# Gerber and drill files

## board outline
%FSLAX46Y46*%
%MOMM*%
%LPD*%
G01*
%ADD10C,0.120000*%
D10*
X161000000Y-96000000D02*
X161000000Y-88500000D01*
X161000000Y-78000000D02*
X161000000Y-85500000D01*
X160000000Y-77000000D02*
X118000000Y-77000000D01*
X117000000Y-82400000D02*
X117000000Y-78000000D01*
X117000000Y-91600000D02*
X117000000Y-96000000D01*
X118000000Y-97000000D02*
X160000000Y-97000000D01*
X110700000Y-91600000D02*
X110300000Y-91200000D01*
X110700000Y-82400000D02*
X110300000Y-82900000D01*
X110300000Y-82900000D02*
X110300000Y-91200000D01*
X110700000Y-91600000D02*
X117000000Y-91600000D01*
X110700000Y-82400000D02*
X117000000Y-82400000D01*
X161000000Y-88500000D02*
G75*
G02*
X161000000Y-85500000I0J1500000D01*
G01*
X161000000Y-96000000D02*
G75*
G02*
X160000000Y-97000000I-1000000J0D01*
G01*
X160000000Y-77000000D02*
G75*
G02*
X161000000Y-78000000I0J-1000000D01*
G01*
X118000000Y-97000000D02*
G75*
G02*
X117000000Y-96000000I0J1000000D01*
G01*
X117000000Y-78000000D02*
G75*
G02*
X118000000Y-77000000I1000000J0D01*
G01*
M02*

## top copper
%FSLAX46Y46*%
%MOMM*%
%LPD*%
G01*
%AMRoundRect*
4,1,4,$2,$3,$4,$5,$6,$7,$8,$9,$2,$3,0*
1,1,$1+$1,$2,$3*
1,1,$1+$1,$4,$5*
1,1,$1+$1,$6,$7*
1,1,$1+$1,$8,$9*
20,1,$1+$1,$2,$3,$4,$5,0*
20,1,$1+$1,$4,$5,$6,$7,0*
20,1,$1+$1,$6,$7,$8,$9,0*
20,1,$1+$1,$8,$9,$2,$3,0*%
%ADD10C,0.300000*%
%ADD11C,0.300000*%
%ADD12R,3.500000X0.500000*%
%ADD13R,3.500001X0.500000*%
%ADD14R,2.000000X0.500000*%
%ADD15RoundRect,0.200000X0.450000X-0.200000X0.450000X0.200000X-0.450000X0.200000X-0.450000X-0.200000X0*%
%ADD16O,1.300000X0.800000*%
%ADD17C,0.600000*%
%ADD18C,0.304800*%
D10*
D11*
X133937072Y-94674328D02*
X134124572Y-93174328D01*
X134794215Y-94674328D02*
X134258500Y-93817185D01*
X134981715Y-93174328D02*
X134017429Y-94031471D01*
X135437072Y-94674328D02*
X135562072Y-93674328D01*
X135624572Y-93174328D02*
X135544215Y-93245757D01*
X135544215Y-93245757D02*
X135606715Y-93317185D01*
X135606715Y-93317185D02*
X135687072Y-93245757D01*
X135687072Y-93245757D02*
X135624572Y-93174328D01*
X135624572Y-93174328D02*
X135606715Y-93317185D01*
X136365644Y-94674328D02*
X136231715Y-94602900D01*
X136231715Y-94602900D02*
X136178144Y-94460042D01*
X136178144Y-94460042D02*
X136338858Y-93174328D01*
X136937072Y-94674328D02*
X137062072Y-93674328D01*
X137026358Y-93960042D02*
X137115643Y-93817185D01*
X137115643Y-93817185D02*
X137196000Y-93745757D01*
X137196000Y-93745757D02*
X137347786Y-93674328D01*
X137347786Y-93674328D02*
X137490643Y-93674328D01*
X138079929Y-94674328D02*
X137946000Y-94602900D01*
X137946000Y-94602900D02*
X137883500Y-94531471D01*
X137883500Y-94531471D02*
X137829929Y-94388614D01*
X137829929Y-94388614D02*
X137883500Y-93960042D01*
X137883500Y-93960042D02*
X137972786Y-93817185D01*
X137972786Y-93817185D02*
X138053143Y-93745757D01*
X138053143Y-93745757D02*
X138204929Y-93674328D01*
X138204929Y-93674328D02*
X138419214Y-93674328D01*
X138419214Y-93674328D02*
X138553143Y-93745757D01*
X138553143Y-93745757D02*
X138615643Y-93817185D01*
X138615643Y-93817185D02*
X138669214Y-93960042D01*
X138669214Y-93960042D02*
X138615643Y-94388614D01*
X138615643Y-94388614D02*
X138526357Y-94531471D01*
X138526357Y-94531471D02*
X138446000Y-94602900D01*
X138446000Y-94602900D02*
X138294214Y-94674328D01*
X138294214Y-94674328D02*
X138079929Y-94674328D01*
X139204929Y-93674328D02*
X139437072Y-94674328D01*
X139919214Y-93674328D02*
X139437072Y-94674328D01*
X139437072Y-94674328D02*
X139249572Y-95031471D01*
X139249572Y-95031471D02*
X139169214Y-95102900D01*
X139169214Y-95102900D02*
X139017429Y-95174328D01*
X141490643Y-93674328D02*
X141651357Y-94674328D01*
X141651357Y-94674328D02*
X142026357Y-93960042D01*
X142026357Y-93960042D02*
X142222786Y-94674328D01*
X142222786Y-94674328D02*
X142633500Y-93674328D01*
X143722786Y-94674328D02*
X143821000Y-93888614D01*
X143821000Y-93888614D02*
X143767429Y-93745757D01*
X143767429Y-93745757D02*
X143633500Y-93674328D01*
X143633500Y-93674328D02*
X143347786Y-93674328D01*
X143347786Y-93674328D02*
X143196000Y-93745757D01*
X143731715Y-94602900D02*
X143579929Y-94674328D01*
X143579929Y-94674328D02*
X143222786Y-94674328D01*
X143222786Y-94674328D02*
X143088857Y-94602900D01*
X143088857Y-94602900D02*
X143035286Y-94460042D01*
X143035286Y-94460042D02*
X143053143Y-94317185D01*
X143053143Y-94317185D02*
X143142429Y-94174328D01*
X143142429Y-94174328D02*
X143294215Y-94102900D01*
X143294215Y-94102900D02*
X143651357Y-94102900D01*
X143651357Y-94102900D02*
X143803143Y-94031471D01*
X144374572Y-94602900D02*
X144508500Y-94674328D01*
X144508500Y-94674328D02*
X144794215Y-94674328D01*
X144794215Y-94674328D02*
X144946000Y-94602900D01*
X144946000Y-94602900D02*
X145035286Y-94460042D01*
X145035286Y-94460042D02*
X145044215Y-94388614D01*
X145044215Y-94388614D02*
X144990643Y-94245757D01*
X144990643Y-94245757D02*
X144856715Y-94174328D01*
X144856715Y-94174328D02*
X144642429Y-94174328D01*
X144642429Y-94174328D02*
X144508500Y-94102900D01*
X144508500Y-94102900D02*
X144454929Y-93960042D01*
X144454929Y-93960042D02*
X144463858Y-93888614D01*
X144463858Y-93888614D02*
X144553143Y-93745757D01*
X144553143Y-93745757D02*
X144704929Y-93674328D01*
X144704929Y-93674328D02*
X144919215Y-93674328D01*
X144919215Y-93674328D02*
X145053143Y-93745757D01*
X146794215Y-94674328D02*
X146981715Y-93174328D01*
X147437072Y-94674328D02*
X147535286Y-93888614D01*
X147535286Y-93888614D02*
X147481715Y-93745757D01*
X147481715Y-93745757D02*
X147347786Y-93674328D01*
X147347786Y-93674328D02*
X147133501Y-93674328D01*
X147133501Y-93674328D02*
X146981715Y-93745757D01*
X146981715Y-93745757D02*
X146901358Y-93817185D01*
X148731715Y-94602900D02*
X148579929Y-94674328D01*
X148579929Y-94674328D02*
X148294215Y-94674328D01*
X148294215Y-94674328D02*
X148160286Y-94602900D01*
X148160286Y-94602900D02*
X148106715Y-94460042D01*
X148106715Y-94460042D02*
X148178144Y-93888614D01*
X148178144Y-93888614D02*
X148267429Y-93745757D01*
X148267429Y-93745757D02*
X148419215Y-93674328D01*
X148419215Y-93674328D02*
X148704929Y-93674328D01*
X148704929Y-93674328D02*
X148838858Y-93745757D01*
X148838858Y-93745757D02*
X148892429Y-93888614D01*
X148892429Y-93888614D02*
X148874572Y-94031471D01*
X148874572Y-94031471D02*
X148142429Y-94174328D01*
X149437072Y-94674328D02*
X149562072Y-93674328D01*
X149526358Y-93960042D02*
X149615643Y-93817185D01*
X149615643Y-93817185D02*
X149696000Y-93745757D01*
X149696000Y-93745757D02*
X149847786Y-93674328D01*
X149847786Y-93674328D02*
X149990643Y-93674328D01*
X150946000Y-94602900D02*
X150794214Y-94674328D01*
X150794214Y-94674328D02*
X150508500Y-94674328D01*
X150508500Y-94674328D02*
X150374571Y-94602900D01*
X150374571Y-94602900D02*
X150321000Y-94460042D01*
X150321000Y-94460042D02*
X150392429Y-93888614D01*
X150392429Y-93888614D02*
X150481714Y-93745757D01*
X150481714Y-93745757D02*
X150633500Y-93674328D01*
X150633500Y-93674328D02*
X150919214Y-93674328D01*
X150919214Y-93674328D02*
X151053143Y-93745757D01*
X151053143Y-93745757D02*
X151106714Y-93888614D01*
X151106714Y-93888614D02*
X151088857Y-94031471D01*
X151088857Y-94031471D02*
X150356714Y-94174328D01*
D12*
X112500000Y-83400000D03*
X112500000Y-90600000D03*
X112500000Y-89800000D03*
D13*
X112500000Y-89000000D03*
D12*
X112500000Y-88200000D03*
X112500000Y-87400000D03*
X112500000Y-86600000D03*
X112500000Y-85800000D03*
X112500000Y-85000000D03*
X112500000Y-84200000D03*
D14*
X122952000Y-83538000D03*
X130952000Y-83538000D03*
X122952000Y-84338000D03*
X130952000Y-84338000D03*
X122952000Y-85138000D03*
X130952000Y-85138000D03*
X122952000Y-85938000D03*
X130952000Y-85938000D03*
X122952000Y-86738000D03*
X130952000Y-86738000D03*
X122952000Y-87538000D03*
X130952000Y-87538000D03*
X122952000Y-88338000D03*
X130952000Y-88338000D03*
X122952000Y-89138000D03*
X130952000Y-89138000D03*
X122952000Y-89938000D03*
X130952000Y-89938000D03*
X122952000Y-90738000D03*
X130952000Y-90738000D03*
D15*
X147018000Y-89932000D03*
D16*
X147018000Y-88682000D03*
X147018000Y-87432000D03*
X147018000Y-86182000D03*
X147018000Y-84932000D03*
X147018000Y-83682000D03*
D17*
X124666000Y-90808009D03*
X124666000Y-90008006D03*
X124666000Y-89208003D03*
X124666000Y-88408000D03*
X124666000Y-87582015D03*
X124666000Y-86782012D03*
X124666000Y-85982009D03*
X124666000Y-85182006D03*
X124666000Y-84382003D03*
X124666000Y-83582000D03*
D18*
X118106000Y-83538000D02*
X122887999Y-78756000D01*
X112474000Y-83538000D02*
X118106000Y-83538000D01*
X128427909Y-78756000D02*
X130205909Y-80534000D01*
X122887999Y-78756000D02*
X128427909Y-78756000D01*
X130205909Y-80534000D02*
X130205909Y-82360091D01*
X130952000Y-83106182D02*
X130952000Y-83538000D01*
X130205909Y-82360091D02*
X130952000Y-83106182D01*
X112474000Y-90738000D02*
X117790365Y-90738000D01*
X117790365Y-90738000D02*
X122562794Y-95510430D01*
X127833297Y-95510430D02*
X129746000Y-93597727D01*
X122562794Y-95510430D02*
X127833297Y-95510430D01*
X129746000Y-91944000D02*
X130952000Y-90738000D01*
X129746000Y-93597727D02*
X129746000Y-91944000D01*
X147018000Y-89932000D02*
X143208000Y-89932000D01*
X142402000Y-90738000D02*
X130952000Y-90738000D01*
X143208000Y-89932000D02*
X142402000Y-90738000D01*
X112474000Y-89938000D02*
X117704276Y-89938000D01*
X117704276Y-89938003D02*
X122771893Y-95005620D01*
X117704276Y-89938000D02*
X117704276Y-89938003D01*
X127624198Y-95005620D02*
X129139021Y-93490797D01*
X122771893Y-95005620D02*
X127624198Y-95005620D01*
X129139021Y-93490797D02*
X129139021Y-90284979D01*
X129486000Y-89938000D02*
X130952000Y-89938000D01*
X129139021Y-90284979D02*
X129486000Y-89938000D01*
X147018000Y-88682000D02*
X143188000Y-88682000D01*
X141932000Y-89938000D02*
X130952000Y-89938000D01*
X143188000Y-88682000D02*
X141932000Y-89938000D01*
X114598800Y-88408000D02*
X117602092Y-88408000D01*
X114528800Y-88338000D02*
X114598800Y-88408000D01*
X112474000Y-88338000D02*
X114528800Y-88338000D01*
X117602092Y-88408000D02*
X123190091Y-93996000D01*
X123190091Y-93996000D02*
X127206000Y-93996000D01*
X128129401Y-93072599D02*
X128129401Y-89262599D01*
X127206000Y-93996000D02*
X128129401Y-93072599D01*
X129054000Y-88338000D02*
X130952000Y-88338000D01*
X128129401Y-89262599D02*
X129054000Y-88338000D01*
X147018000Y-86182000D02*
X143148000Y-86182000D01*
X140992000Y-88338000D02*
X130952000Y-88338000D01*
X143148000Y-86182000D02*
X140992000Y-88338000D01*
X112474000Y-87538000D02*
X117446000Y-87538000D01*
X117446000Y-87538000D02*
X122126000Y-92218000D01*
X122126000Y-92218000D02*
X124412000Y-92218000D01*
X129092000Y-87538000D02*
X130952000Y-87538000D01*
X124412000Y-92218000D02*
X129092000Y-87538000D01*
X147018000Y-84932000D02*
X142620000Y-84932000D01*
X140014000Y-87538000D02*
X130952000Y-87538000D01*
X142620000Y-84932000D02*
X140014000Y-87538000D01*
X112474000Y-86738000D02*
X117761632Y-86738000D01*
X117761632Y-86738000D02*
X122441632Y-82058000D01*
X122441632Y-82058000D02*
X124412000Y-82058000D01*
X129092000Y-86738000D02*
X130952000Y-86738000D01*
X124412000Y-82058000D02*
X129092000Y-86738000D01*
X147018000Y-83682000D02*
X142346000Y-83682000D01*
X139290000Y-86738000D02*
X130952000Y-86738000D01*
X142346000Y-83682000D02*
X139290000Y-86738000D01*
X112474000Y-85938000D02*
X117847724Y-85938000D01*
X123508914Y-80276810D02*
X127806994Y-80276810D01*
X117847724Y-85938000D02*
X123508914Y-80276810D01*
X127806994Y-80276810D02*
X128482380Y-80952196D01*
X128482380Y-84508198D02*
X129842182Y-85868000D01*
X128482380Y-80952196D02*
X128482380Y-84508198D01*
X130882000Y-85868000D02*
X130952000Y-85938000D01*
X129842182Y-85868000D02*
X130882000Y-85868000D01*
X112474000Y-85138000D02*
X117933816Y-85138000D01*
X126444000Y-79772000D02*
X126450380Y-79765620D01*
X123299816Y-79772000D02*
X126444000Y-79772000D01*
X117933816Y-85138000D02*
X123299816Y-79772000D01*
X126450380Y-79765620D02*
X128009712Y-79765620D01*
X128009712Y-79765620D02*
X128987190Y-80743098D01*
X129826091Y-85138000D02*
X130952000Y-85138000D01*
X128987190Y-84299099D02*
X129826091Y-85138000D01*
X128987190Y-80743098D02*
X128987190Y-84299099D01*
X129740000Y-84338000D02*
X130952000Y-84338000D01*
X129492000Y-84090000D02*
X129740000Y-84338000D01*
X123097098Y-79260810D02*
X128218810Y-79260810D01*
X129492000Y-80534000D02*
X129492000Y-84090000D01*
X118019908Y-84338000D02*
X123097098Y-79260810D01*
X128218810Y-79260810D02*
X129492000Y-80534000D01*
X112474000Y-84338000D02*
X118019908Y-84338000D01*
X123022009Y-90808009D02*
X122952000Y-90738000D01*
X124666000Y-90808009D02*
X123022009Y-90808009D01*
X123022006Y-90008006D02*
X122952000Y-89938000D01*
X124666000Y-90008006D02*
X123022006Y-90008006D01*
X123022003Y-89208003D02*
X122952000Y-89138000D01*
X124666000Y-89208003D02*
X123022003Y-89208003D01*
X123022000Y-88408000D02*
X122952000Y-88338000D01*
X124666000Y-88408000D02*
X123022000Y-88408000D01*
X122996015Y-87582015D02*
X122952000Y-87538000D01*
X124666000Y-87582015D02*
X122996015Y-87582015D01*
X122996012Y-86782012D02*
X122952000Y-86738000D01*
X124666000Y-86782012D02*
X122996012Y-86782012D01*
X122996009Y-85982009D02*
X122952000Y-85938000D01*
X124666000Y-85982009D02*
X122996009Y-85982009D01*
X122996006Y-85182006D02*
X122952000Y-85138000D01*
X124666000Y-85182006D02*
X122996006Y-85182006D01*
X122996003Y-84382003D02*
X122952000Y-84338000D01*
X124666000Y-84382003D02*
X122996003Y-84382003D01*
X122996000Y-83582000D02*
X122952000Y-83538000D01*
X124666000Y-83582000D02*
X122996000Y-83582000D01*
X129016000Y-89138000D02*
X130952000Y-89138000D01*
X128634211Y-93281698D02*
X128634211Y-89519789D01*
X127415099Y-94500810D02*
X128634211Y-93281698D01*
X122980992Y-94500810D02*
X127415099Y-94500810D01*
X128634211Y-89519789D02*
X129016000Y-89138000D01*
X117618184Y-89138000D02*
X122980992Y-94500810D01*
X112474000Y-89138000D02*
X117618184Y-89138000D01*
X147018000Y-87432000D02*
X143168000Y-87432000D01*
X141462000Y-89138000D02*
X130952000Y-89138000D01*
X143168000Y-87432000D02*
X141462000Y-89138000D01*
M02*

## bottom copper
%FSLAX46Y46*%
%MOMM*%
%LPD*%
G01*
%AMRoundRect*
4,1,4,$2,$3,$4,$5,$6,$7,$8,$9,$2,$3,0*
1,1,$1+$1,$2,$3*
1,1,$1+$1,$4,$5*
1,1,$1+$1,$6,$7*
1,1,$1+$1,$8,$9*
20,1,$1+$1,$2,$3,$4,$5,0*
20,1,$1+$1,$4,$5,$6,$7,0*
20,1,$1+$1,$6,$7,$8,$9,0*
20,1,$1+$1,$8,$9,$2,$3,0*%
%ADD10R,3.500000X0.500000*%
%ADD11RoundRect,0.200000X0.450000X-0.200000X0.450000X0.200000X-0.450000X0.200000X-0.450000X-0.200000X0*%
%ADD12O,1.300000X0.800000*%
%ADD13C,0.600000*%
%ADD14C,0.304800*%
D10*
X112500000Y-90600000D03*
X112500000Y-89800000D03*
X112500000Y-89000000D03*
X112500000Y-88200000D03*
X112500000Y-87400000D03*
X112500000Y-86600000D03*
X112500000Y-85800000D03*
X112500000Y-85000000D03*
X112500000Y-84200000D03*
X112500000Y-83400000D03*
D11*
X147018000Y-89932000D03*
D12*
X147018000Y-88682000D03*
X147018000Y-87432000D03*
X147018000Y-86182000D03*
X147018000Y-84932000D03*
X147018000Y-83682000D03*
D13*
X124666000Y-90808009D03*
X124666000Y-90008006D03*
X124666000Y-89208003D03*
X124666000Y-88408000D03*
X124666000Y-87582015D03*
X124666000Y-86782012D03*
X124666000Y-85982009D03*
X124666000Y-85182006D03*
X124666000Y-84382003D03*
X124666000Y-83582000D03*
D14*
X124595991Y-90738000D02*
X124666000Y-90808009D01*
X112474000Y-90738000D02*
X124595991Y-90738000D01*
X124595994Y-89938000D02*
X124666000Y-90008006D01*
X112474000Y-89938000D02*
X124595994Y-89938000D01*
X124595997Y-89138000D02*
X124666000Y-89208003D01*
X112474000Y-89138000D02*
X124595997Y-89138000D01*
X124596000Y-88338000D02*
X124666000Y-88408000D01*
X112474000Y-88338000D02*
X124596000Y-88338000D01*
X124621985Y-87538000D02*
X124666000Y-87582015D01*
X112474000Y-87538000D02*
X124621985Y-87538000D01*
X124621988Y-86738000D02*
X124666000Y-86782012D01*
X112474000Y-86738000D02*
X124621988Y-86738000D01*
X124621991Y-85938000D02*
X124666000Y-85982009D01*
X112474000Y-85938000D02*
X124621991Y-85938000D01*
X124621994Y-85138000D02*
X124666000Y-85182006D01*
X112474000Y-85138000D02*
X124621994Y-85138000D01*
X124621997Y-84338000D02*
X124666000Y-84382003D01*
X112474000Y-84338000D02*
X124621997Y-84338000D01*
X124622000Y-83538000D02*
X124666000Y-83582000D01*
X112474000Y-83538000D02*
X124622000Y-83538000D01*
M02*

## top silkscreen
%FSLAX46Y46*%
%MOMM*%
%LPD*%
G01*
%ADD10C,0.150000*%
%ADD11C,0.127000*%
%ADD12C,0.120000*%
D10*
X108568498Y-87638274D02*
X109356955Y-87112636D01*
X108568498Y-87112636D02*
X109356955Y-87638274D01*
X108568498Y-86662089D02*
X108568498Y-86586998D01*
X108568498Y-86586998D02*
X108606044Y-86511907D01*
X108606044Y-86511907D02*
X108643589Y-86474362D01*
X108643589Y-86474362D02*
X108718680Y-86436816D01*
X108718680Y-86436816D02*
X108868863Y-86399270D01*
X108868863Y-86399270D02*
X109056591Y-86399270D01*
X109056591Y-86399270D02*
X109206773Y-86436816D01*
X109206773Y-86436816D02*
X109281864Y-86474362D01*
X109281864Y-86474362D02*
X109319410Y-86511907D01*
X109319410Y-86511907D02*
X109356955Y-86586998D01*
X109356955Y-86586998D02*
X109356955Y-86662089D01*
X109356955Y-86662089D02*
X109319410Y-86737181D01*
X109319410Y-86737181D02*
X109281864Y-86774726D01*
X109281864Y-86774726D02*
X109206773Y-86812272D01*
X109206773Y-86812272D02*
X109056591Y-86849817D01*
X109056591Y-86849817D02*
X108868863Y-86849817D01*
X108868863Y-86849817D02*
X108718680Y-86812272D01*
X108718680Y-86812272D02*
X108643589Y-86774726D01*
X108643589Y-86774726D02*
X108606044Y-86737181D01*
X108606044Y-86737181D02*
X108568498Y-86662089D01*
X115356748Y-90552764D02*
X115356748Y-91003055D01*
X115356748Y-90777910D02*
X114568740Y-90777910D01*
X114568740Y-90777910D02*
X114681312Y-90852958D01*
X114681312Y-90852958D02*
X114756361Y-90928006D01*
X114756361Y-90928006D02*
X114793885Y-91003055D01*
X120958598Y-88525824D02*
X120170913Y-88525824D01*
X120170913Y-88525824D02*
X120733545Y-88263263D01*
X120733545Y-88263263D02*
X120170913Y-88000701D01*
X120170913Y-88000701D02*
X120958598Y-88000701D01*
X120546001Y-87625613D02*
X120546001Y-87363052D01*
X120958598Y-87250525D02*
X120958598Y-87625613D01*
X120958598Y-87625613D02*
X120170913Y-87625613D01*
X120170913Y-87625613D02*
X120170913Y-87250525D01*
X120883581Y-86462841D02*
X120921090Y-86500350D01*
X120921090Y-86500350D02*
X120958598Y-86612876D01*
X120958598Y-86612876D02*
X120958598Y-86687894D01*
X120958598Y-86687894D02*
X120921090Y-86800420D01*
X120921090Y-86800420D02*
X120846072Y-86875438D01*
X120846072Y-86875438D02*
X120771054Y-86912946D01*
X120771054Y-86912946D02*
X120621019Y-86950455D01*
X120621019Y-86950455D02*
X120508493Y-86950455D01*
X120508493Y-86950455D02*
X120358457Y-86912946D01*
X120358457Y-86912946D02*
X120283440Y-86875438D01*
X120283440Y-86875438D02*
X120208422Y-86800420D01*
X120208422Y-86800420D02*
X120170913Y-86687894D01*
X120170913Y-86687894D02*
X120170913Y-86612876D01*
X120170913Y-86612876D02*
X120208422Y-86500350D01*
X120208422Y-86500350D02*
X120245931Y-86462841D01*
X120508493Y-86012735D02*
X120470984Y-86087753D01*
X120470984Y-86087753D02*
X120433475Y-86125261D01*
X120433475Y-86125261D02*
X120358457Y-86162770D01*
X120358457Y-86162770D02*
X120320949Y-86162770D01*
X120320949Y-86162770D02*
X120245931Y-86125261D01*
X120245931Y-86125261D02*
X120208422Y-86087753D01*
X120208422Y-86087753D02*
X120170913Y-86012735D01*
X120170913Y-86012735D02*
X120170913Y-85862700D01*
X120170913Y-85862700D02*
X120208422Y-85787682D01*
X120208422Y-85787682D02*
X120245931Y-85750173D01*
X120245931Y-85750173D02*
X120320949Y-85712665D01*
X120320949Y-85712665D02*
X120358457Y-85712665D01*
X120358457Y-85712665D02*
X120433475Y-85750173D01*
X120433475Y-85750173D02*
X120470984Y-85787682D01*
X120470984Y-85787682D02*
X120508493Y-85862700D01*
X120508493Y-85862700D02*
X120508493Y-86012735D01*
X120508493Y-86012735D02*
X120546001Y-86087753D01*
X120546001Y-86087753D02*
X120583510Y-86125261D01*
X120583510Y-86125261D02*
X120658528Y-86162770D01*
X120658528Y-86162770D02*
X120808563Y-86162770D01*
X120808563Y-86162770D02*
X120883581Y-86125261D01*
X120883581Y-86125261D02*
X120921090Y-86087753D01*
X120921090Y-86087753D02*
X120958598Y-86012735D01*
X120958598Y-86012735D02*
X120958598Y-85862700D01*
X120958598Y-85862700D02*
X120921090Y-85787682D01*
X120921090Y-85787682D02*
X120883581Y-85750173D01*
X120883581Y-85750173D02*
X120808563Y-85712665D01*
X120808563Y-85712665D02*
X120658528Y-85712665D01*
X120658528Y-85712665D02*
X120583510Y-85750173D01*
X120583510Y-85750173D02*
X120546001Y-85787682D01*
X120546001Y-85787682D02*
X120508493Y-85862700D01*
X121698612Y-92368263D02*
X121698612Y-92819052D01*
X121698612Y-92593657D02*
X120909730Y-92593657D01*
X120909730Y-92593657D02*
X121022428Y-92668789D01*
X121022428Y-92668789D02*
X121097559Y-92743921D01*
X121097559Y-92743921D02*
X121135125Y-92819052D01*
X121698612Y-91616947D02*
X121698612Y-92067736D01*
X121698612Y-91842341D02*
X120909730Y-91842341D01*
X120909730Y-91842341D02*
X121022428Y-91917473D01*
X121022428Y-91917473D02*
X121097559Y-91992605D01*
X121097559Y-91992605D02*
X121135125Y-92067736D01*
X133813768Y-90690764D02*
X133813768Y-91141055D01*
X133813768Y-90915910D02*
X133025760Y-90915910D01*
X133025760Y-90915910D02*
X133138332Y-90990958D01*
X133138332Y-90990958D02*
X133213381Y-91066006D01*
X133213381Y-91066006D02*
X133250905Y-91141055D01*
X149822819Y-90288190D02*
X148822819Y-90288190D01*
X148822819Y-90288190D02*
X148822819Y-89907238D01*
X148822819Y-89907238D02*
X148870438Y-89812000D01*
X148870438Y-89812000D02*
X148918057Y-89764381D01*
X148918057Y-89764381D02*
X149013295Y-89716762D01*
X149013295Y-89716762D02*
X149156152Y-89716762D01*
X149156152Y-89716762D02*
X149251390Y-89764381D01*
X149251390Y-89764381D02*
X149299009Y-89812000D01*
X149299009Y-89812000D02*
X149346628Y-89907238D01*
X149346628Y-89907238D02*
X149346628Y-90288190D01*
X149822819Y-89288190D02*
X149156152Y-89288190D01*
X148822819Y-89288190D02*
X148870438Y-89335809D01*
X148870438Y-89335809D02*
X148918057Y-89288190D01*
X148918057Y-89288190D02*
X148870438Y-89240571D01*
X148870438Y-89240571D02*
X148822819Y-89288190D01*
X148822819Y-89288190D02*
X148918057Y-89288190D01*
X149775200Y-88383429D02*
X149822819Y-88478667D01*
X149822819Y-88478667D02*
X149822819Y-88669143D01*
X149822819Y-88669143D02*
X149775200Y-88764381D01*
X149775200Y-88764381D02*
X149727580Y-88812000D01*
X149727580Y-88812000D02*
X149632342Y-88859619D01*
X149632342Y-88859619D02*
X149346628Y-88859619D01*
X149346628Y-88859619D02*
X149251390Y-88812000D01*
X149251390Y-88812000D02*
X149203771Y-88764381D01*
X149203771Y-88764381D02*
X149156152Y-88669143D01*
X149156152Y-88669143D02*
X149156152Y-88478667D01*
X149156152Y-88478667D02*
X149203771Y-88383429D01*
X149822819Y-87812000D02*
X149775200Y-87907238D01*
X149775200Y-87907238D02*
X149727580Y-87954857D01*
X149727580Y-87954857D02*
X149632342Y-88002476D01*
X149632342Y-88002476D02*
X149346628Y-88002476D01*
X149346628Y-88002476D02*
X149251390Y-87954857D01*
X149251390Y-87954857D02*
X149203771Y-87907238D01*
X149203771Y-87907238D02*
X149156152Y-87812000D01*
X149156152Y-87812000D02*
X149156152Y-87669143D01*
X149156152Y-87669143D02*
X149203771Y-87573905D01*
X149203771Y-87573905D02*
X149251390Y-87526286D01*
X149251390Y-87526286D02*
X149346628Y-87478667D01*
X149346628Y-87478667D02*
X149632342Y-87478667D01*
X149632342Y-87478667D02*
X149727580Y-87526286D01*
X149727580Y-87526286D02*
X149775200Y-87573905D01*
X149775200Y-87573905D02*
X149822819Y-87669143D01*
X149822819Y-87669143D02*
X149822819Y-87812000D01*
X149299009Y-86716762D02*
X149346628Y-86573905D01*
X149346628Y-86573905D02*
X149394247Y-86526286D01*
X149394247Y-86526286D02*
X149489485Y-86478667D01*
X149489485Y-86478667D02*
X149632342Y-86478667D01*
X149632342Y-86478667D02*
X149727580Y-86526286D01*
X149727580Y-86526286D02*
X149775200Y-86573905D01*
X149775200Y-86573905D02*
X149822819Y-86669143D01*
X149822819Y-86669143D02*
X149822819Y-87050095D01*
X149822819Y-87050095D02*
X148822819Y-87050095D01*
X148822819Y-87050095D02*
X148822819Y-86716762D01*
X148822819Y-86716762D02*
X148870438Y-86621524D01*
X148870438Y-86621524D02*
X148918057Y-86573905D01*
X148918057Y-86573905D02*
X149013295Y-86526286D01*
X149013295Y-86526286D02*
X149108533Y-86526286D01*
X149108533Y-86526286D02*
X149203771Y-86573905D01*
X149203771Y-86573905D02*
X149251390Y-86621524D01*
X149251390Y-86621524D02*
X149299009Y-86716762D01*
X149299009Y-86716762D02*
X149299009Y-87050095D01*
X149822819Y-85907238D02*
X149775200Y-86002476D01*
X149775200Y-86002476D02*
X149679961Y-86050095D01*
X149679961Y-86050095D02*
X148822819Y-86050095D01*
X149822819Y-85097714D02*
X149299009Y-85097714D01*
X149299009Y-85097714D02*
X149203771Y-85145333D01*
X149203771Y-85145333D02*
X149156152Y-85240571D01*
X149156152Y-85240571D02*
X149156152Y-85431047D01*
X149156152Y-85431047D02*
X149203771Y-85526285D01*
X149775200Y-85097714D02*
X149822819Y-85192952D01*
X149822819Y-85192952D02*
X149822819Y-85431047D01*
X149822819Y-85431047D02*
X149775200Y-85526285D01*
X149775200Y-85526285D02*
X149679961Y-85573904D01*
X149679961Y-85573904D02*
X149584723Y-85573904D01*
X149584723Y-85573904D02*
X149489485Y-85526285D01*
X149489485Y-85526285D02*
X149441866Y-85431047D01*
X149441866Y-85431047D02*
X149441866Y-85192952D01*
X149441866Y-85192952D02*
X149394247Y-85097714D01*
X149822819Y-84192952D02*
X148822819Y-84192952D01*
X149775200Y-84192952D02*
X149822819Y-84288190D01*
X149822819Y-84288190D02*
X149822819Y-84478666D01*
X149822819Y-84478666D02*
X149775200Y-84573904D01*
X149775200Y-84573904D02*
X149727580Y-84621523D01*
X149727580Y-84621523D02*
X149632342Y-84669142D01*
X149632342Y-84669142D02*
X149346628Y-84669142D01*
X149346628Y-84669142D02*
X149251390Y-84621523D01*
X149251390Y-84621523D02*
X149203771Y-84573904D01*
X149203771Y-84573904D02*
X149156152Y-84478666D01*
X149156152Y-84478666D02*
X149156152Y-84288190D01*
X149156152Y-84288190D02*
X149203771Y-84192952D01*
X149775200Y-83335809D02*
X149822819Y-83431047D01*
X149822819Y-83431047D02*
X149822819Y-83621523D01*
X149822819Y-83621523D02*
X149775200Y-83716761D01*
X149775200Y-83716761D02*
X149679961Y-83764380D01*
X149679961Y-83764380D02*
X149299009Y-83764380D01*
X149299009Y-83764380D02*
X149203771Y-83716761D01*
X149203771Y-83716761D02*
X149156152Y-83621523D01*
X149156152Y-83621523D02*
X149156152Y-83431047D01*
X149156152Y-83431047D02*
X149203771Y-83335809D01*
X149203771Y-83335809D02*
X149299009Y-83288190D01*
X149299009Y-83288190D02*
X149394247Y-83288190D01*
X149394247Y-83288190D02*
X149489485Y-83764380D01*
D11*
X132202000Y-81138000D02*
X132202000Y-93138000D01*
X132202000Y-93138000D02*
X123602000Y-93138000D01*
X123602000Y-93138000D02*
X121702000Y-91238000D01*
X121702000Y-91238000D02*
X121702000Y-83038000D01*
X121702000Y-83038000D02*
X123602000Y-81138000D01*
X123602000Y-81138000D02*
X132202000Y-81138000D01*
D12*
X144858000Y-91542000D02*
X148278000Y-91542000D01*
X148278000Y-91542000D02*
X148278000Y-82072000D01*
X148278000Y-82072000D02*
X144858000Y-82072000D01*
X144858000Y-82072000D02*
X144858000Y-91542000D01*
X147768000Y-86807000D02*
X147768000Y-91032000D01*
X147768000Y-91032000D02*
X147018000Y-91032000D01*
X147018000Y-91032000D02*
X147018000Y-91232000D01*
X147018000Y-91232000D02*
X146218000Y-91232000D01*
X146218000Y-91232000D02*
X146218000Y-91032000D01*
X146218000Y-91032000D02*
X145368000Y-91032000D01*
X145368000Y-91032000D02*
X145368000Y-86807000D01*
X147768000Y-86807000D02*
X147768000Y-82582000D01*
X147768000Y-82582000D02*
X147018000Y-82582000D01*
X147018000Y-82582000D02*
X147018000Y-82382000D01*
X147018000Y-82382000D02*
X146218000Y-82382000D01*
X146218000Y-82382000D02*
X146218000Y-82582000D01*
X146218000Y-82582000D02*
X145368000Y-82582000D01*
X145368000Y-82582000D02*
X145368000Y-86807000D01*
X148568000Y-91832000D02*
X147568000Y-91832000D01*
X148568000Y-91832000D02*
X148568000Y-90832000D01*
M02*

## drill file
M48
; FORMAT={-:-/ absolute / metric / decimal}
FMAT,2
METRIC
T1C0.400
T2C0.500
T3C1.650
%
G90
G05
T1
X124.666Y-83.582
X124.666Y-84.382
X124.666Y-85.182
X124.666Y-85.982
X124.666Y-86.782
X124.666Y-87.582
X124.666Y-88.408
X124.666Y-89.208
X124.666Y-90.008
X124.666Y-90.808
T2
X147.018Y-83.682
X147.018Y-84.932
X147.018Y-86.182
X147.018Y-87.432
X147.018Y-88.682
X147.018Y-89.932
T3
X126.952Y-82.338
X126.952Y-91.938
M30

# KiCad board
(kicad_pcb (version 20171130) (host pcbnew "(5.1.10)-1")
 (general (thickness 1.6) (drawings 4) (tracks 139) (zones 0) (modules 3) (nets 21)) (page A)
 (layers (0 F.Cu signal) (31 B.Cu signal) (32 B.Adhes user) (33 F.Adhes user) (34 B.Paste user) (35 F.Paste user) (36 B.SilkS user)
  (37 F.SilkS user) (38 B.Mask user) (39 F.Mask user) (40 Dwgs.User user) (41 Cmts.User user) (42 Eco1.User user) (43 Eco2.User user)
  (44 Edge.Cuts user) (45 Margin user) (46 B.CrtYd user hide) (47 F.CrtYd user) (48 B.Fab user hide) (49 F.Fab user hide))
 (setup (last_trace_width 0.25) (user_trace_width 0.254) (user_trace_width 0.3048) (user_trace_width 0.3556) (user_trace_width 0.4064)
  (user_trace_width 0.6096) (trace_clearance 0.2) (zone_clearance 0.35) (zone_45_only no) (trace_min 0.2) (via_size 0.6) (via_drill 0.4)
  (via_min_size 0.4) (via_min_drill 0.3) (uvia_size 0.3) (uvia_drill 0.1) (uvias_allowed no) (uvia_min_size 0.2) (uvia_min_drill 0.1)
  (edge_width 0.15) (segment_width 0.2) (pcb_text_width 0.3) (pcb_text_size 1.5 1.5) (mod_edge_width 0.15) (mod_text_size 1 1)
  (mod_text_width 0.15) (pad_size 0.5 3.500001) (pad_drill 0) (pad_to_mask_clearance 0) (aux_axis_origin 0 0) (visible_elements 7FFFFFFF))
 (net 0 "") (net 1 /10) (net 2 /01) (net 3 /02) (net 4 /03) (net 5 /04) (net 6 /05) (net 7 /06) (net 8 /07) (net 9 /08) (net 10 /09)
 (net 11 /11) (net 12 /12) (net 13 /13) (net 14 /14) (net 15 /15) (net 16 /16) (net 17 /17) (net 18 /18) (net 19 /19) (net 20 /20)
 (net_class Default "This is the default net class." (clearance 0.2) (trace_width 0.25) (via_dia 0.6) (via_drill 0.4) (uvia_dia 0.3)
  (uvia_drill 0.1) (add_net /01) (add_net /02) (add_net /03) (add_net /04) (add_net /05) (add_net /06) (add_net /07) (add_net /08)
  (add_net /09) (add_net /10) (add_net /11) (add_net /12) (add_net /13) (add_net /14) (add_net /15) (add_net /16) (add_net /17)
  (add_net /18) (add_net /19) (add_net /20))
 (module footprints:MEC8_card (layer F.Cu) (at 112.5 87 90)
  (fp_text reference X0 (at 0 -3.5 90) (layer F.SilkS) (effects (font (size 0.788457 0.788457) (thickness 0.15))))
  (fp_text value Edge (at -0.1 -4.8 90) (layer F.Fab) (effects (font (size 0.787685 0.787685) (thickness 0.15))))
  (fp_line (start -9 48.5) (end -1.5 48.5) (layer Edge.Cuts) (width 0.12))
  (fp_line (start 9 48.5) (end 1.5 48.5) (layer Edge.Cuts) (width 0.12))
  (fp_line (start 10 47.5) (end 10 5.5) (layer Edge.Cuts) (width 0.12))
  (fp_line (start 4.6 4.5) (end 9 4.5) (layer Edge.Cuts) (width 0.12))
  (fp_line (start -4.6 4.5) (end -9 4.5) (layer Edge.Cuts) (width 0.12))
  (fp_line (start -10 5.5) (end -10 47.5) (layer Edge.Cuts) (width 0.12))
  (fp_line (start -4.6 -1.8) (end -4.2 -2.2) (layer Edge.Cuts) (width 0.12))
  (fp_line (start 4.6 -1.8) (end 4.1 -2.2) (layer Edge.Cuts) (width 0.12))
  (fp_line (start 4.1 -2.2) (end -4.2 -2.2) (layer Edge.Cuts) (width 0.12))
  (fp_line (start -4.6 -1.8) (end -4.6 4.5) (layer Edge.Cuts) (width 0.12))
  (fp_line (start 4.6 -1.8) (end 4.6 4.5) (layer Edge.Cuts) (width 0.12))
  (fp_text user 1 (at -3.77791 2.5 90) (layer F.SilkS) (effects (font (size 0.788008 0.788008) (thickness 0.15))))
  (fp_arc (start 0 48.5) (end 1.5 48.5) (angle -180) (layer Edge.Cuts) (width 0.12))
  (fp_arc (start -9 47.5) (end -10 47.5) (angle -90) (layer Edge.Cuts) (width 0.12))
  (fp_arc (start 9 47.5) (end 9 48.5) (angle -90) (layer Edge.Cuts) (width 0.12))
  (fp_arc (start -9 5.5) (end -9 4.5) (angle -90) (layer Edge.Cuts) (width 0.12))
  (fp_arc (start 9 5.5) (end 10 5.5) (angle -90) (layer Edge.Cuts) (width 0.12))
  (pad 10 smd rect (at 3.6 0 90) (size 0.5 3.5) (layers F.Cu F.Paste F.Mask) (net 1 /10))
  (pad 1 smd rect (at -3.6 0 90) (size 0.5 3.5) (layers F.Cu F.Paste F.Mask) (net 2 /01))
  (pad 2 smd rect (at -2.8 0 90) (size 0.5 3.5) (layers F.Cu F.Paste F.Mask) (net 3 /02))
  (pad 3 smd rect (at -2 0 90) (size 0.5 3.500001) (layers F.Cu F.Paste F.Mask) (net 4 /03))
  (pad 4 smd rect (at -1.2 0 90) (size 0.5 3.5) (layers F.Cu F.Paste F.Mask) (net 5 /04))
  (pad 5 smd rect (at -0.4 0 90) (size 0.5 3.5) (layers F.Cu F.Paste F.Mask) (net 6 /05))
  (pad 6 smd rect (at 0.4 0 90) (size 0.5 3.5) (layers F.Cu F.Paste F.Mask) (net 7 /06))
  (pad 7 smd rect (at 1.2 0 90) (size 0.5 3.5) (layers F.Cu F.Paste F.Mask) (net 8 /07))
  (pad 8 smd rect (at 2 0 90) (size 0.5 3.5) (layers F.Cu F.Paste F.Mask) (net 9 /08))
  (pad 9 smd rect (at 2.8 0 90) (size 0.5 3.5) (layers F.Cu F.Paste F.Mask) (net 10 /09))
  (pad 11 smd rect (at -3.6 0 90) (size 0.5 3.5) (layers B.Cu B.Paste B.Mask) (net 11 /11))
  (pad 12 smd rect (at -2.8 0 90) (size 0.5 3.5) (layers B.Cu B.Paste B.Mask) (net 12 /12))
  (pad 13 smd rect (at -2 0 90) (size 0.5 3.5) (layers B.Cu B.Paste B.Mask) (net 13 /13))
  (pad 14 smd rect (at -1.2 0 90) (size 0.5 3.5) (layers B.Cu B.Paste B.Mask) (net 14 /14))
  (pad 15 smd rect (at -0.4 0 90) (size 0.5 3.5) (layers B.Cu B.Paste B.Mask) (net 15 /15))
  (pad 16 smd rect (at 0.4 0 90) (size 0.5 3.5) (layers B.Cu B.Paste B.Mask) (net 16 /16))
  (pad 17 smd rect (at 1.2 0 90) (size 0.5 3.5) (layers B.Cu B.Paste B.Mask) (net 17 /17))
  (pad 18 smd rect (at 2 0 90) (size 0.5 3.5) (layers B.Cu B.Paste B.Mask) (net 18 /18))
  (pad 19 smd rect (at 2.8 0 90) (size 0.5 3.5) (layers B.Cu B.Paste B.Mask) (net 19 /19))
  (pad 20 smd rect (at 3.6 0 90) (size 0.5 3.5) (layers B.Cu B.Paste B.Mask) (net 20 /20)))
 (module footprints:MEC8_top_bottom (layer F.Cu) (at 126.952 87.138 90)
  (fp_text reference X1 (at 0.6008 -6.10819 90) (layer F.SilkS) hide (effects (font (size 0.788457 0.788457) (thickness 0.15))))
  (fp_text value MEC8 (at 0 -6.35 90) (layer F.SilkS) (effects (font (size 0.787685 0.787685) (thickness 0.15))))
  (fp_line (start 6 5.25) (end -6 5.25) (layer F.SilkS) (width 0.127))
  (fp_line (start -6 5.25) (end -6 -3.35) (layer F.SilkS) (width 0.127))
  (fp_line (start -6 -3.35) (end -4.1 -5.25) (layer F.SilkS) (width 0.127))
  (fp_line (start -4.1 -5.25) (end 4.1 -5.25) (layer F.SilkS) (width 0.127))
  (fp_line (start 4.1 -5.25) (end 6 -3.35) (layer F.SilkS) (width 0.127))
  (fp_line (start 6 -3.35) (end 6 5.25) (layer F.SilkS) (width 0.127))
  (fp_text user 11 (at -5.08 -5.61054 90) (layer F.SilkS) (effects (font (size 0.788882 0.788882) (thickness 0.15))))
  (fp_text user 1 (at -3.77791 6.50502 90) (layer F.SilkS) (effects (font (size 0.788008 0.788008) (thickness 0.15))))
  (pad None np_thru_hole circle (at 4.8 0 90) (size 1.65 1.65) (drill 1.65) (layers *.Cu *.Mask))
  (pad None np_thru_hole circle (at -4.8 0 90) (size 1.65 1.65) (drill 1.65) (layers *.Cu *.Mask))
  (pad 20 smd rect (at 3.6 -4 90) (size 0.5 2) (layers F.Cu F.Paste F.Mask) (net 20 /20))
  (pad 10 smd rect (at 3.6 4 90) (size 0.5 2) (layers F.Cu F.Paste F.Mask) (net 1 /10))
  (pad 19 smd rect (at 2.8 -4 90) (size 0.5 2) (layers F.Cu F.Paste F.Mask) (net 19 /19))
  (pad 9 smd rect (at 2.8 4 90) (size 0.5 2) (layers F.Cu F.Paste F.Mask) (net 10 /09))
  (pad 18 smd rect (at 2 -4 90) (size 0.5 2) (layers F.Cu F.Paste F.Mask) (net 18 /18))
  (pad 8 smd rect (at 2 4 90) (size 0.5 2) (layers F.Cu F.Paste F.Mask) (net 9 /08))
  (pad 17 smd rect (at 1.2 -4 90) (size 0.5 2) (layers F.Cu F.Paste F.Mask) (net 17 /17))
  (pad 7 smd rect (at 1.2 4 90) (size 0.5 2) (layers F.Cu F.Paste F.Mask) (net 8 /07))
  (pad 16 smd rect (at 0.4 -4 90) (size 0.5 2) (layers F.Cu F.Paste F.Mask) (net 16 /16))
  (pad 6 smd rect (at 0.4 4 90) (size 0.5 2) (layers F.Cu F.Paste F.Mask) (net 7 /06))
  (pad 15 smd rect (at -0.4 -4 90) (size 0.5 2) (layers F.Cu F.Paste F.Mask) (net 15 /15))
  (pad 5 smd rect (at -0.4 4 90) (size 0.5 2) (layers F.Cu F.Paste F.Mask) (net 6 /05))
  (pad 14 smd rect (at -1.2 -4 90) (size 0.5 2) (layers F.Cu F.Paste F.Mask) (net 14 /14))
  (pad 4 smd rect (at -1.2 4 90) (size 0.5 2) (layers F.Cu F.Paste F.Mask) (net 5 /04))
  (pad 13 smd rect (at -2 -4 90) (size 0.5 2) (layers F.Cu F.Paste F.Mask) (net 13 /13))
  (pad 3 smd rect (at -2 4 90) (size 0.5 2) (layers F.Cu F.Paste F.Mask) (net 4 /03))
  (pad 12 smd rect (at -2.8 -4 90) (size 0.5 2) (layers F.Cu F.Paste F.Mask) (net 12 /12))
  (pad 2 smd rect (at -2.8 4 90) (size 0.5 2) (layers F.Cu F.Paste F.Mask) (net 3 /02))
  (pad 11 smd rect (at -3.6 -4 90) (size 0.5 2) (layers F.Cu F.Paste F.Mask) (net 11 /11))
  (pad 1 smd rect (at -3.6 4 90) (size 0.5 2) (layers F.Cu F.Paste F.Mask) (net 2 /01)))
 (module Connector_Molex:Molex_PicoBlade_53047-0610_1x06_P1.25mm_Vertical (layer F.Cu) (at 147.018 89.932 90)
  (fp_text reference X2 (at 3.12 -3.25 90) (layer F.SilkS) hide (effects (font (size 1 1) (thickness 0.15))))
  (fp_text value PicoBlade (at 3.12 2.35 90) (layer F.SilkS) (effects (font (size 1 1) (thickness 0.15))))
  (fp_line (start -1.61 -2.16) (end -1.61 1.26) (layer F.SilkS) (width 0.12))
  (fp_line (start -1.61 1.26) (end 7.86 1.26) (layer F.SilkS) (width 0.12))
  (fp_line (start 7.86 1.26) (end 7.86 -2.16) (layer F.SilkS) (width 0.12))
  (fp_line (start 7.86 -2.16) (end -1.61 -2.16) (layer F.SilkS) (width 0.12))
  (fp_line (start 3.125 0.75) (end -1.1 0.75) (layer F.SilkS) (width 0.12))
  (fp_line (start -1.1 0.75) (end -1.1 0) (layer F.SilkS) (width 0.12))
  (fp_line (start -1.1 0) (end -1.3 0) (layer F.SilkS) (width 0.12))
  (fp_line (start -1.3 0) (end -1.3 -0.8) (layer F.SilkS) (width 0.12))
  (fp_line (start -1.3 -0.8) (end -1.1 -0.8) (layer F.SilkS) (width 0.12))
  (fp_line (start -1.1 -0.8) (end -1.1 -1.65) (layer F.SilkS) (width 0.12))
  (fp_line (start -1.1 -1.65) (end 3.125 -1.65) (layer F.SilkS) (width 0.12))
  (fp_line (start 3.125 0.75) (end 7.35 0.75) (layer F.SilkS) (width 0.12))
  (fp_line (start 7.35 0.75) (end 7.35 0) (layer F.SilkS) (width 0.12))
  (fp_line (start 7.35 0) (end 7.55 0) (layer F.SilkS) (width 0.12))
  (fp_line (start 7.55 0) (end 7.55 -0.8) (layer F.SilkS) (width 0.12))
  (fp_line (start 7.55 -0.8) (end 7.35 -0.8) (layer F.SilkS) (width 0.12))
  (fp_line (start 7.35 -0.8) (end 7.35 -1.65) (layer F.SilkS) (width 0.12))
  (fp_line (start 7.35 -1.65) (end 3.125 -1.65) (layer F.SilkS) (width 0.12))
  (fp_line (start -1.9 1.55) (end -1.9 0.55) (layer F.SilkS) (width 0.12))
  (fp_line (start -1.9 1.55) (end -0.9 1.55) (layer F.SilkS) (width 0.12))
  (pad 1 thru_hole roundrect (at 0 0 90) (size 0.8 1.3) (drill 0.5) (layers *.Cu *.Mask) (roundrect_rratio 0.25) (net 2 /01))
  (pad 2 thru_hole oval (at 1.25 0 90) (size 0.8 1.3) (drill 0.5) (layers *.Cu *.Mask) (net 3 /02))
  (pad 3 thru_hole oval (at 2.5 0 90) (size 0.8 1.3) (drill 0.5) (layers *.Cu *.Mask) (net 4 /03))
  (pad 4 thru_hole oval (at 3.75 0 90) (size 0.8 1.3) (drill 0.5) (layers *.Cu *.Mask) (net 5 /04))
  (pad 5 thru_hole oval (at 5 0 90) (size 0.8 1.3) (drill 0.5) (layers *.Cu *.Mask) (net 6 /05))
  (pad 6 thru_hole oval (at 6.25 0 90) (size 0.8 1.3) (drill 0.5) (layers *.Cu *.Mask) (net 7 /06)))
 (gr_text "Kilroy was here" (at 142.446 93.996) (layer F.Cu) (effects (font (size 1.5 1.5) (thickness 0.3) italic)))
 (segment (start 118.106 83.538) (end 122.887999 78.756) (width 0.3048) (layer F.Cu) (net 1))
 (segment (start 112.474 83.538) (end 118.106 83.538) (width 0.3048) (layer F.Cu) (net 1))
 (segment (start 128.427909 78.756) (end 130.205909 80.534) (width 0.3048) (layer F.Cu) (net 1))
 (segment (start 122.887999 78.756) (end 128.427909 78.756) (width 0.3048) (layer F.Cu) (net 1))
 (segment (start 130.205909 80.534) (end 130.205909 82.360091) (width 0.3048) (layer F.Cu) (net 1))
 (segment (start 130.952 83.106182) (end 130.952 83.538) (width 0.3048) (layer F.Cu) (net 1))
 (segment (start 130.205909 82.360091) (end 130.952 83.106182) (width 0.3048) (layer F.Cu) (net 1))
 (segment (start 112.474 90.738) (end 117.790365 90.738) (width 0.3048) (layer F.Cu) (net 2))
 (segment (start 117.790365 90.738) (end 122.562794 95.51043) (width 0.3048) (layer F.Cu) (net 2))
 (segment (start 127.833297 95.51043) (end 129.746 93.597727) (width 0.3048) (layer F.Cu) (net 2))
 (segment (start 122.562794 95.51043) (end 127.833297 95.51043) (width 0.3048) (layer F.Cu) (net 2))
 (segment (start 129.746 91.944) (end 130.952 90.738) (width 0.3048) (layer F.Cu) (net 2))
 (segment (start 129.746 93.597727) (end 129.746 91.944) (width 0.3048) (layer F.Cu) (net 2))
 (segment (start 147.018 89.932) (end 143.208 89.932) (width 0.3048) (layer F.Cu) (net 2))
 (segment (start 142.402 90.738) (end 130.952 90.738) (width 0.3048) (layer F.Cu) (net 2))
 (segment (start 143.208 89.932) (end 142.402 90.738) (width 0.3048) (layer F.Cu) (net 2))
 (segment (start 112.474 89.938) (end 117.704276 89.938) (width 0.3048) (layer F.Cu) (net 3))
 (segment (start 117.704276 89.938003) (end 122.771893 95.00562) (width 0.3048) (layer F.Cu) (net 3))
 (segment (start 117.704276 89.938) (end 117.704276 89.938003) (width 0.3048) (layer F.Cu) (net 3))
 (segment (start 127.624198 95.00562) (end 129.139021 93.490797) (width 0.3048) (layer F.Cu) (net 3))
 (segment (start 122.771893 95.00562) (end 127.624198 95.00562) (width 0.3048) (layer F.Cu) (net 3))
 (segment (start 129.139021 93.490797) (end 129.139021 90.284979) (width 0.3048) (layer F.Cu) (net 3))
 (segment (start 129.486 89.938) (end 130.952 89.938) (width 0.3048) (layer F.Cu) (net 3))
 (segment (start 129.139021 90.284979) (end 129.486 89.938) (width 0.3048) (layer F.Cu) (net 3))
 (segment (start 147.018 88.682) (end 143.188 88.682) (width 0.3048) (layer F.Cu) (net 3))
 (segment (start 141.932 89.938) (end 130.952 89.938) (width 0.3048) (layer F.Cu) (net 3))
 (segment (start 143.188 88.682) (end 141.932 89.938) (width 0.3048) (layer F.Cu) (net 3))
 (segment (start 114.5988 88.408) (end 117.602092 88.408) (width 0.3048) (layer F.Cu) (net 5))
 (segment (start 114.5288 88.338) (end 114.5988 88.408) (width 0.3048) (layer F.Cu) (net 5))
 (segment (start 112.474 88.338) (end 114.5288 88.338) (width 0.3048) (layer F.Cu) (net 5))
 (segment (start 117.602092 88.408) (end 123.190091 93.996) (width 0.3048) (layer F.Cu) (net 5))
 (segment (start 123.190091 93.996) (end 127.206 93.996) (width 0.3048) (layer F.Cu) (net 5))
 (segment (start 128.129401 93.072599) (end 128.129401 89.262599) (width 0.3048) (layer F.Cu) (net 5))
 (segment (start 127.206 93.996) (end 128.129401 93.072599) (width 0.3048) (layer F.Cu) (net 5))
 (segment (start 129.054 88.338) (end 130.952 88.338) (width 0.3048) (layer F.Cu) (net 5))
 (segment (start 128.129401 89.262599) (end 129.054 88.338) (width 0.3048) (layer F.Cu) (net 5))
 (segment (start 147.018 86.182) (end 143.148 86.182) (width 0.3048) (layer F.Cu) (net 5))
 (segment (start 140.992 88.338) (end 130.952 88.338) (width 0.3048) (layer F.Cu) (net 5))
 (segment (start 143.148 86.182) (end 140.992 88.338) (width 0.3048) (layer F.Cu) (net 5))
 (segment (start 112.474 87.538) (end 117.446 87.538) (width 0.3048) (layer F.Cu) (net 6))
 (segment (start 117.446 87.538) (end 122.126 92.218) (width 0.3048) (layer F.Cu) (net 6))
 (segment (start 122.126 92.218) (end 124.412 92.218) (width 0.3048) (layer F.Cu) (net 6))
 (segment (start 129.092 87.538) (end 130.952 87.538) (width 0.3048) (layer F.Cu) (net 6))
 (segment (start 124.412 92.218) (end 129.092 87.538) (width 0.3048) (layer F.Cu) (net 6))
 (segment (start 147.018 84.932) (end 142.62 84.932) (width 0.3048) (layer F.Cu) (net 6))
 (segment (start 140.014 87.538) (end 130.952 87.538) (width 0.3048) (layer F.Cu) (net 6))
 (segment (start 142.62 84.932) (end 140.014 87.538) (width 0.3048) (layer F.Cu) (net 6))
 (segment (start 112.474 86.738) (end 117.761632 86.738) (width 0.3048) (layer F.Cu) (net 7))
 (segment (start 117.761632 86.738) (end 122.441632 82.058) (width 0.3048) (layer F.Cu) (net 7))
 (segment (start 122.441632 82.058) (end 124.412 82.058) (width 0.3048) (layer F.Cu) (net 7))
 (segment (start 129.092 86.738) (end 130.952 86.738) (width 0.3048) (layer F.Cu) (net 7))
 (segment (start 124.412 82.058) (end 129.092 86.738) (width 0.3048) (layer F.Cu) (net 7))
 (segment (start 147.018 83.682) (end 142.346 83.682) (width 0.3048) (layer F.Cu) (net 7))
 (segment (start 139.29 86.738) (end 130.952 86.738) (width 0.3048) (layer F.Cu) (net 7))
 (segment (start 142.346 83.682) (end 139.29 86.738) (width 0.3048) (layer F.Cu) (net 7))
 (segment (start 112.474 85.938) (end 117.847724 85.938) (width 0.3048) (layer F.Cu) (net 8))
 (segment (start 123.508914 80.27681) (end 127.806994 80.27681) (width 0.3048) (layer F.Cu) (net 8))
 (segment (start 117.847724 85.938) (end 123.508914 80.27681) (width 0.3048) (layer F.Cu) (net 8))
 (segment (start 127.806994 80.27681) (end 128.48238 80.952196) (width 0.3048) (layer F.Cu) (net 8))
 (segment (start 128.48238 84.508198) (end 129.842182 85.868) (width 0.3048) (layer F.Cu) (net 8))
 (segment (start 128.48238 80.952196) (end 128.48238 84.508198) (width 0.3048) (layer F.Cu) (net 8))
 (segment (start 130.882 85.868) (end 130.952 85.938) (width 0.3048) (layer F.Cu) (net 8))
 (segment (start 129.842182 85.868) (end 130.882 85.868) (width 0.3048) (layer F.Cu) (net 8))
 (segment (start 112.474 85.138) (end 117.933816 85.138) (width 0.3048) (layer F.Cu) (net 9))
 (segment (start 126.444 79.772) (end 126.45038 79.76562) (width 0.3048) (layer F.Cu) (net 9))
 (segment (start 123.299816 79.772) (end 126.444 79.772) (width 0.3048) (layer F.Cu) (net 9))
 (segment (start 117.933816 85.138) (end 123.299816 79.772) (width 0.3048) (layer F.Cu) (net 9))
 (segment (start 126.45038 79.76562) (end 128.009712 79.76562) (width 0.3048) (layer F.Cu) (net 9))
 (segment (start 128.009712 79.76562) (end 128.98719 80.743098) (width 0.3048) (layer F.Cu) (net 9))
 (segment (start 129.826091 85.138) (end 130.952 85.138) (width 0.3048) (layer F.Cu) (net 9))
 (segment (start 128.98719 84.299099) (end 129.826091 85.138) (width 0.3048) (layer F.Cu) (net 9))
 (segment (start 128.98719 80.743098) (end 128.98719 84.299099) (width 0.3048) (layer F.Cu) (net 9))
 (segment (start 129.74 84.338) (end 130.952 84.338) (width 0.3048) (layer F.Cu) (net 10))
 (segment (start 129.492 84.09) (end 129.74 84.338) (width 0.3048) (layer F.Cu) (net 10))
 (segment (start 123.097098 79.26081) (end 128.21881 79.26081) (width 0.3048) (layer F.Cu) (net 10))
 (segment (start 129.492 80.534) (end 129.492 84.09) (width 0.3048) (layer F.Cu) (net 10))
 (segment (start 118.019908 84.338) (end 123.097098 79.26081) (width 0.3048) (layer F.Cu) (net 10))
 (segment (start 128.21881 79.26081) (end 129.492 80.534) (width 0.3048) (layer F.Cu) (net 10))
 (segment (start 112.474 84.338) (end 118.019908 84.338) (width 0.3048) (layer F.Cu) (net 10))
 (via (at 124.666 90.808009) (size 0.6) (drill 0.4) (layers F.Cu B.Cu) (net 11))
 (segment (start 124.595991 90.738) (end 124.666 90.808009) (width 0.3048) (layer B.Cu) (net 11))
 (segment (start 112.474 90.738) (end 124.595991 90.738) (width 0.3048) (layer B.Cu) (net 11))
 (segment (start 123.022009 90.808009) (end 122.952 90.738) (width 0.3048) (layer F.Cu) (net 11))
 (segment (start 124.666 90.808009) (end 123.022009 90.808009) (width 0.3048) (layer F.Cu) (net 11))
 (via (at 124.666 90.008006) (size 0.6) (drill 0.4) (layers F.Cu B.Cu) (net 12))
 (segment (start 124.595994 89.938) (end 124.666 90.008006) (width 0.3048) (layer B.Cu) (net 12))
 (segment (start 112.474 89.938) (end 124.595994 89.938) (width 0.3048) (layer B.Cu) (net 12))
 (segment (start 123.022006 90.008006) (end 122.952 89.938) (width 0.3048) (layer F.Cu) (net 12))
 (segment (start 124.666 90.008006) (end 123.022006 90.008006) (width 0.3048) (layer F.Cu) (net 12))
 (segment (start 124.595997 89.138) (end 124.666 89.208003) (width 0.3048) (layer B.Cu) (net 13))
 (via (at 124.666 89.208003) (size 0.6) (drill 0.4) (layers F.Cu B.Cu) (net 13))
 (segment (start 112.474 89.138) (end 124.595997 89.138) (width 0.3048) (layer B.Cu) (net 13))
 (segment (start 123.022003 89.208003) (end 122.952 89.138) (width 0.3048) (layer F.Cu) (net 13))
 (segment (start 124.666 89.208003) (end 123.022003 89.208003) (width 0.3048) (layer F.Cu) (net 13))
 (via (at 124.666 88.408) (size 0.6) (drill 0.4) (layers F.Cu B.Cu) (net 14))
 (segment (start 124.596 88.338) (end 124.666 88.408) (width 0.3048) (layer B.Cu) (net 14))
 (segment (start 112.474 88.338) (end 124.596 88.338) (width 0.3048) (layer B.Cu) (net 14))
 (segment (start 123.022 88.408) (end 122.952 88.338) (width 0.3048) (layer F.Cu) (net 14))
 (segment (start 124.666 88.408) (end 123.022 88.408) (width 0.3048) (layer F.Cu) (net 14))
 (via (at 124.666 87.582015) (size 0.6) (drill 0.4) (layers F.Cu B.Cu) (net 15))
 (segment (start 124.621985 87.538) (end 124.666 87.582015) (width 0.3048) (layer B.Cu) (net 15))
 (segment (start 112.474 87.538) (end 124.621985 87.538) (width 0.3048) (layer B.Cu) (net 15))
 (segment (start 122.996015 87.582015) (end 122.952 87.538) (width 0.3048) (layer F.Cu) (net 15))
 (segment (start 124.666 87.582015) (end 122.996015 87.582015) (width 0.3048) (layer F.Cu) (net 15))
 (via (at 124.666 86.782012) (size 0.6) (drill 0.4) (layers F.Cu B.Cu) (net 16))
 (segment (start 124.621988 86.738) (end 124.666 86.782012) (width 0.3048) (layer B.Cu) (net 16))
 (segment (start 112.474 86.738) (end 124.621988 86.738) (width 0.3048) (layer B.Cu) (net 16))
 (segment (start 122.996012 86.782012) (end 122.952 86.738) (width 0.3048) (layer F.Cu) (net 16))
 (segment (start 124.666 86.782012) (end 122.996012 86.782012) (width 0.3048) (layer F.Cu) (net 16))
 (via (at 124.666 85.982009) (size 0.6) (drill 0.4) (layers F.Cu B.Cu) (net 17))
 (segment (start 124.621991 85.938) (end 124.666 85.982009) (width 0.3048) (layer B.Cu) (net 17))
 (segment (start 112.474 85.938) (end 124.621991 85.938) (width 0.3048) (layer B.Cu) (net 17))
 (segment (start 122.996009 85.982009) (end 122.952 85.938) (width 0.3048) (layer F.Cu) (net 17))
 (segment (start 124.666 85.982009) (end 122.996009 85.982009) (width 0.3048) (layer F.Cu) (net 17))
 (via (at 124.666 85.182006) (size 0.6) (drill 0.4) (layers F.Cu B.Cu) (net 18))
 (segment (start 124.621994 85.138) (end 124.666 85.182006) (width 0.3048) (layer B.Cu) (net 18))
 (segment (start 112.474 85.138) (end 124.621994 85.138) (width 0.3048) (layer B.Cu) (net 18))
 (segment (start 122.996006 85.182006) (end 122.952 85.138) (width 0.3048) (layer F.Cu) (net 18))
 (segment (start 124.666 85.182006) (end 122.996006 85.182006) (width 0.3048) (layer F.Cu) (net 18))
 (via (at 124.666 84.382003) (size 0.6) (drill 0.4) (layers F.Cu B.Cu) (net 19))
 (segment (start 124.621997 84.338) (end 124.666 84.382003) (width 0.3048) (layer B.Cu) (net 19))
 (segment (start 112.474 84.338) (end 124.621997 84.338) (width 0.3048) (layer B.Cu) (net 19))
 (segment (start 122.996003 84.382003) (end 122.952 84.338) (width 0.3048) (layer F.Cu) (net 19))
 (segment (start 124.666 84.382003) (end 122.996003 84.382003) (width 0.3048) (layer F.Cu) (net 19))
 (via (at 124.666 83.582) (size 0.6) (drill 0.4) (layers F.Cu B.Cu) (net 20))
 (segment (start 124.622 83.538) (end 124.666 83.582) (width 0.3048) (layer B.Cu) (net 20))
 (segment (start 112.474 83.538) (end 124.622 83.538) (width 0.3048) (layer B.Cu) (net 20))
 (segment (start 122.996 83.582) (end 122.952 83.538) (width 0.3048) (layer F.Cu) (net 20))
 (segment (start 124.666 83.582) (end 122.996 83.582) (width 0.3048) (layer F.Cu) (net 20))
 (segment (start 129.016 89.138) (end 130.952 89.138) (width 0.3048) (layer F.Cu) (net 4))
 (segment (start 128.634211 93.281698) (end 128.634211 89.519789) (width 0.3048) (layer F.Cu) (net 4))
 (segment (start 127.415099 94.50081) (end 128.634211 93.281698) (width 0.3048) (layer F.Cu) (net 4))
 (segment (start 122.980992 94.50081) (end 127.415099 94.50081) (width 0.3048) (layer F.Cu) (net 4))
 (segment (start 128.634211 89.519789) (end 129.016 89.138) (width 0.3048) (layer F.Cu) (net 4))
 (segment (start 117.618184 89.138) (end 122.980992 94.50081) (width 0.3048) (layer F.Cu) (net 4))
 (segment (start 112.474 89.138) (end 117.618184 89.138) (width 0.3048) (layer F.Cu) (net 4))
 (segment (start 147.018 87.432) (end 143.168 87.432) (width 0.3048) (layer F.Cu) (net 4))
 (segment (start 141.462 89.138) (end 130.952 89.138) (width 0.3048) (layer F.Cu) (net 4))
 (segment (start 143.168 87.432) (end 141.462 89.138) (width 0.3048) (layer F.Cu) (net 4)))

